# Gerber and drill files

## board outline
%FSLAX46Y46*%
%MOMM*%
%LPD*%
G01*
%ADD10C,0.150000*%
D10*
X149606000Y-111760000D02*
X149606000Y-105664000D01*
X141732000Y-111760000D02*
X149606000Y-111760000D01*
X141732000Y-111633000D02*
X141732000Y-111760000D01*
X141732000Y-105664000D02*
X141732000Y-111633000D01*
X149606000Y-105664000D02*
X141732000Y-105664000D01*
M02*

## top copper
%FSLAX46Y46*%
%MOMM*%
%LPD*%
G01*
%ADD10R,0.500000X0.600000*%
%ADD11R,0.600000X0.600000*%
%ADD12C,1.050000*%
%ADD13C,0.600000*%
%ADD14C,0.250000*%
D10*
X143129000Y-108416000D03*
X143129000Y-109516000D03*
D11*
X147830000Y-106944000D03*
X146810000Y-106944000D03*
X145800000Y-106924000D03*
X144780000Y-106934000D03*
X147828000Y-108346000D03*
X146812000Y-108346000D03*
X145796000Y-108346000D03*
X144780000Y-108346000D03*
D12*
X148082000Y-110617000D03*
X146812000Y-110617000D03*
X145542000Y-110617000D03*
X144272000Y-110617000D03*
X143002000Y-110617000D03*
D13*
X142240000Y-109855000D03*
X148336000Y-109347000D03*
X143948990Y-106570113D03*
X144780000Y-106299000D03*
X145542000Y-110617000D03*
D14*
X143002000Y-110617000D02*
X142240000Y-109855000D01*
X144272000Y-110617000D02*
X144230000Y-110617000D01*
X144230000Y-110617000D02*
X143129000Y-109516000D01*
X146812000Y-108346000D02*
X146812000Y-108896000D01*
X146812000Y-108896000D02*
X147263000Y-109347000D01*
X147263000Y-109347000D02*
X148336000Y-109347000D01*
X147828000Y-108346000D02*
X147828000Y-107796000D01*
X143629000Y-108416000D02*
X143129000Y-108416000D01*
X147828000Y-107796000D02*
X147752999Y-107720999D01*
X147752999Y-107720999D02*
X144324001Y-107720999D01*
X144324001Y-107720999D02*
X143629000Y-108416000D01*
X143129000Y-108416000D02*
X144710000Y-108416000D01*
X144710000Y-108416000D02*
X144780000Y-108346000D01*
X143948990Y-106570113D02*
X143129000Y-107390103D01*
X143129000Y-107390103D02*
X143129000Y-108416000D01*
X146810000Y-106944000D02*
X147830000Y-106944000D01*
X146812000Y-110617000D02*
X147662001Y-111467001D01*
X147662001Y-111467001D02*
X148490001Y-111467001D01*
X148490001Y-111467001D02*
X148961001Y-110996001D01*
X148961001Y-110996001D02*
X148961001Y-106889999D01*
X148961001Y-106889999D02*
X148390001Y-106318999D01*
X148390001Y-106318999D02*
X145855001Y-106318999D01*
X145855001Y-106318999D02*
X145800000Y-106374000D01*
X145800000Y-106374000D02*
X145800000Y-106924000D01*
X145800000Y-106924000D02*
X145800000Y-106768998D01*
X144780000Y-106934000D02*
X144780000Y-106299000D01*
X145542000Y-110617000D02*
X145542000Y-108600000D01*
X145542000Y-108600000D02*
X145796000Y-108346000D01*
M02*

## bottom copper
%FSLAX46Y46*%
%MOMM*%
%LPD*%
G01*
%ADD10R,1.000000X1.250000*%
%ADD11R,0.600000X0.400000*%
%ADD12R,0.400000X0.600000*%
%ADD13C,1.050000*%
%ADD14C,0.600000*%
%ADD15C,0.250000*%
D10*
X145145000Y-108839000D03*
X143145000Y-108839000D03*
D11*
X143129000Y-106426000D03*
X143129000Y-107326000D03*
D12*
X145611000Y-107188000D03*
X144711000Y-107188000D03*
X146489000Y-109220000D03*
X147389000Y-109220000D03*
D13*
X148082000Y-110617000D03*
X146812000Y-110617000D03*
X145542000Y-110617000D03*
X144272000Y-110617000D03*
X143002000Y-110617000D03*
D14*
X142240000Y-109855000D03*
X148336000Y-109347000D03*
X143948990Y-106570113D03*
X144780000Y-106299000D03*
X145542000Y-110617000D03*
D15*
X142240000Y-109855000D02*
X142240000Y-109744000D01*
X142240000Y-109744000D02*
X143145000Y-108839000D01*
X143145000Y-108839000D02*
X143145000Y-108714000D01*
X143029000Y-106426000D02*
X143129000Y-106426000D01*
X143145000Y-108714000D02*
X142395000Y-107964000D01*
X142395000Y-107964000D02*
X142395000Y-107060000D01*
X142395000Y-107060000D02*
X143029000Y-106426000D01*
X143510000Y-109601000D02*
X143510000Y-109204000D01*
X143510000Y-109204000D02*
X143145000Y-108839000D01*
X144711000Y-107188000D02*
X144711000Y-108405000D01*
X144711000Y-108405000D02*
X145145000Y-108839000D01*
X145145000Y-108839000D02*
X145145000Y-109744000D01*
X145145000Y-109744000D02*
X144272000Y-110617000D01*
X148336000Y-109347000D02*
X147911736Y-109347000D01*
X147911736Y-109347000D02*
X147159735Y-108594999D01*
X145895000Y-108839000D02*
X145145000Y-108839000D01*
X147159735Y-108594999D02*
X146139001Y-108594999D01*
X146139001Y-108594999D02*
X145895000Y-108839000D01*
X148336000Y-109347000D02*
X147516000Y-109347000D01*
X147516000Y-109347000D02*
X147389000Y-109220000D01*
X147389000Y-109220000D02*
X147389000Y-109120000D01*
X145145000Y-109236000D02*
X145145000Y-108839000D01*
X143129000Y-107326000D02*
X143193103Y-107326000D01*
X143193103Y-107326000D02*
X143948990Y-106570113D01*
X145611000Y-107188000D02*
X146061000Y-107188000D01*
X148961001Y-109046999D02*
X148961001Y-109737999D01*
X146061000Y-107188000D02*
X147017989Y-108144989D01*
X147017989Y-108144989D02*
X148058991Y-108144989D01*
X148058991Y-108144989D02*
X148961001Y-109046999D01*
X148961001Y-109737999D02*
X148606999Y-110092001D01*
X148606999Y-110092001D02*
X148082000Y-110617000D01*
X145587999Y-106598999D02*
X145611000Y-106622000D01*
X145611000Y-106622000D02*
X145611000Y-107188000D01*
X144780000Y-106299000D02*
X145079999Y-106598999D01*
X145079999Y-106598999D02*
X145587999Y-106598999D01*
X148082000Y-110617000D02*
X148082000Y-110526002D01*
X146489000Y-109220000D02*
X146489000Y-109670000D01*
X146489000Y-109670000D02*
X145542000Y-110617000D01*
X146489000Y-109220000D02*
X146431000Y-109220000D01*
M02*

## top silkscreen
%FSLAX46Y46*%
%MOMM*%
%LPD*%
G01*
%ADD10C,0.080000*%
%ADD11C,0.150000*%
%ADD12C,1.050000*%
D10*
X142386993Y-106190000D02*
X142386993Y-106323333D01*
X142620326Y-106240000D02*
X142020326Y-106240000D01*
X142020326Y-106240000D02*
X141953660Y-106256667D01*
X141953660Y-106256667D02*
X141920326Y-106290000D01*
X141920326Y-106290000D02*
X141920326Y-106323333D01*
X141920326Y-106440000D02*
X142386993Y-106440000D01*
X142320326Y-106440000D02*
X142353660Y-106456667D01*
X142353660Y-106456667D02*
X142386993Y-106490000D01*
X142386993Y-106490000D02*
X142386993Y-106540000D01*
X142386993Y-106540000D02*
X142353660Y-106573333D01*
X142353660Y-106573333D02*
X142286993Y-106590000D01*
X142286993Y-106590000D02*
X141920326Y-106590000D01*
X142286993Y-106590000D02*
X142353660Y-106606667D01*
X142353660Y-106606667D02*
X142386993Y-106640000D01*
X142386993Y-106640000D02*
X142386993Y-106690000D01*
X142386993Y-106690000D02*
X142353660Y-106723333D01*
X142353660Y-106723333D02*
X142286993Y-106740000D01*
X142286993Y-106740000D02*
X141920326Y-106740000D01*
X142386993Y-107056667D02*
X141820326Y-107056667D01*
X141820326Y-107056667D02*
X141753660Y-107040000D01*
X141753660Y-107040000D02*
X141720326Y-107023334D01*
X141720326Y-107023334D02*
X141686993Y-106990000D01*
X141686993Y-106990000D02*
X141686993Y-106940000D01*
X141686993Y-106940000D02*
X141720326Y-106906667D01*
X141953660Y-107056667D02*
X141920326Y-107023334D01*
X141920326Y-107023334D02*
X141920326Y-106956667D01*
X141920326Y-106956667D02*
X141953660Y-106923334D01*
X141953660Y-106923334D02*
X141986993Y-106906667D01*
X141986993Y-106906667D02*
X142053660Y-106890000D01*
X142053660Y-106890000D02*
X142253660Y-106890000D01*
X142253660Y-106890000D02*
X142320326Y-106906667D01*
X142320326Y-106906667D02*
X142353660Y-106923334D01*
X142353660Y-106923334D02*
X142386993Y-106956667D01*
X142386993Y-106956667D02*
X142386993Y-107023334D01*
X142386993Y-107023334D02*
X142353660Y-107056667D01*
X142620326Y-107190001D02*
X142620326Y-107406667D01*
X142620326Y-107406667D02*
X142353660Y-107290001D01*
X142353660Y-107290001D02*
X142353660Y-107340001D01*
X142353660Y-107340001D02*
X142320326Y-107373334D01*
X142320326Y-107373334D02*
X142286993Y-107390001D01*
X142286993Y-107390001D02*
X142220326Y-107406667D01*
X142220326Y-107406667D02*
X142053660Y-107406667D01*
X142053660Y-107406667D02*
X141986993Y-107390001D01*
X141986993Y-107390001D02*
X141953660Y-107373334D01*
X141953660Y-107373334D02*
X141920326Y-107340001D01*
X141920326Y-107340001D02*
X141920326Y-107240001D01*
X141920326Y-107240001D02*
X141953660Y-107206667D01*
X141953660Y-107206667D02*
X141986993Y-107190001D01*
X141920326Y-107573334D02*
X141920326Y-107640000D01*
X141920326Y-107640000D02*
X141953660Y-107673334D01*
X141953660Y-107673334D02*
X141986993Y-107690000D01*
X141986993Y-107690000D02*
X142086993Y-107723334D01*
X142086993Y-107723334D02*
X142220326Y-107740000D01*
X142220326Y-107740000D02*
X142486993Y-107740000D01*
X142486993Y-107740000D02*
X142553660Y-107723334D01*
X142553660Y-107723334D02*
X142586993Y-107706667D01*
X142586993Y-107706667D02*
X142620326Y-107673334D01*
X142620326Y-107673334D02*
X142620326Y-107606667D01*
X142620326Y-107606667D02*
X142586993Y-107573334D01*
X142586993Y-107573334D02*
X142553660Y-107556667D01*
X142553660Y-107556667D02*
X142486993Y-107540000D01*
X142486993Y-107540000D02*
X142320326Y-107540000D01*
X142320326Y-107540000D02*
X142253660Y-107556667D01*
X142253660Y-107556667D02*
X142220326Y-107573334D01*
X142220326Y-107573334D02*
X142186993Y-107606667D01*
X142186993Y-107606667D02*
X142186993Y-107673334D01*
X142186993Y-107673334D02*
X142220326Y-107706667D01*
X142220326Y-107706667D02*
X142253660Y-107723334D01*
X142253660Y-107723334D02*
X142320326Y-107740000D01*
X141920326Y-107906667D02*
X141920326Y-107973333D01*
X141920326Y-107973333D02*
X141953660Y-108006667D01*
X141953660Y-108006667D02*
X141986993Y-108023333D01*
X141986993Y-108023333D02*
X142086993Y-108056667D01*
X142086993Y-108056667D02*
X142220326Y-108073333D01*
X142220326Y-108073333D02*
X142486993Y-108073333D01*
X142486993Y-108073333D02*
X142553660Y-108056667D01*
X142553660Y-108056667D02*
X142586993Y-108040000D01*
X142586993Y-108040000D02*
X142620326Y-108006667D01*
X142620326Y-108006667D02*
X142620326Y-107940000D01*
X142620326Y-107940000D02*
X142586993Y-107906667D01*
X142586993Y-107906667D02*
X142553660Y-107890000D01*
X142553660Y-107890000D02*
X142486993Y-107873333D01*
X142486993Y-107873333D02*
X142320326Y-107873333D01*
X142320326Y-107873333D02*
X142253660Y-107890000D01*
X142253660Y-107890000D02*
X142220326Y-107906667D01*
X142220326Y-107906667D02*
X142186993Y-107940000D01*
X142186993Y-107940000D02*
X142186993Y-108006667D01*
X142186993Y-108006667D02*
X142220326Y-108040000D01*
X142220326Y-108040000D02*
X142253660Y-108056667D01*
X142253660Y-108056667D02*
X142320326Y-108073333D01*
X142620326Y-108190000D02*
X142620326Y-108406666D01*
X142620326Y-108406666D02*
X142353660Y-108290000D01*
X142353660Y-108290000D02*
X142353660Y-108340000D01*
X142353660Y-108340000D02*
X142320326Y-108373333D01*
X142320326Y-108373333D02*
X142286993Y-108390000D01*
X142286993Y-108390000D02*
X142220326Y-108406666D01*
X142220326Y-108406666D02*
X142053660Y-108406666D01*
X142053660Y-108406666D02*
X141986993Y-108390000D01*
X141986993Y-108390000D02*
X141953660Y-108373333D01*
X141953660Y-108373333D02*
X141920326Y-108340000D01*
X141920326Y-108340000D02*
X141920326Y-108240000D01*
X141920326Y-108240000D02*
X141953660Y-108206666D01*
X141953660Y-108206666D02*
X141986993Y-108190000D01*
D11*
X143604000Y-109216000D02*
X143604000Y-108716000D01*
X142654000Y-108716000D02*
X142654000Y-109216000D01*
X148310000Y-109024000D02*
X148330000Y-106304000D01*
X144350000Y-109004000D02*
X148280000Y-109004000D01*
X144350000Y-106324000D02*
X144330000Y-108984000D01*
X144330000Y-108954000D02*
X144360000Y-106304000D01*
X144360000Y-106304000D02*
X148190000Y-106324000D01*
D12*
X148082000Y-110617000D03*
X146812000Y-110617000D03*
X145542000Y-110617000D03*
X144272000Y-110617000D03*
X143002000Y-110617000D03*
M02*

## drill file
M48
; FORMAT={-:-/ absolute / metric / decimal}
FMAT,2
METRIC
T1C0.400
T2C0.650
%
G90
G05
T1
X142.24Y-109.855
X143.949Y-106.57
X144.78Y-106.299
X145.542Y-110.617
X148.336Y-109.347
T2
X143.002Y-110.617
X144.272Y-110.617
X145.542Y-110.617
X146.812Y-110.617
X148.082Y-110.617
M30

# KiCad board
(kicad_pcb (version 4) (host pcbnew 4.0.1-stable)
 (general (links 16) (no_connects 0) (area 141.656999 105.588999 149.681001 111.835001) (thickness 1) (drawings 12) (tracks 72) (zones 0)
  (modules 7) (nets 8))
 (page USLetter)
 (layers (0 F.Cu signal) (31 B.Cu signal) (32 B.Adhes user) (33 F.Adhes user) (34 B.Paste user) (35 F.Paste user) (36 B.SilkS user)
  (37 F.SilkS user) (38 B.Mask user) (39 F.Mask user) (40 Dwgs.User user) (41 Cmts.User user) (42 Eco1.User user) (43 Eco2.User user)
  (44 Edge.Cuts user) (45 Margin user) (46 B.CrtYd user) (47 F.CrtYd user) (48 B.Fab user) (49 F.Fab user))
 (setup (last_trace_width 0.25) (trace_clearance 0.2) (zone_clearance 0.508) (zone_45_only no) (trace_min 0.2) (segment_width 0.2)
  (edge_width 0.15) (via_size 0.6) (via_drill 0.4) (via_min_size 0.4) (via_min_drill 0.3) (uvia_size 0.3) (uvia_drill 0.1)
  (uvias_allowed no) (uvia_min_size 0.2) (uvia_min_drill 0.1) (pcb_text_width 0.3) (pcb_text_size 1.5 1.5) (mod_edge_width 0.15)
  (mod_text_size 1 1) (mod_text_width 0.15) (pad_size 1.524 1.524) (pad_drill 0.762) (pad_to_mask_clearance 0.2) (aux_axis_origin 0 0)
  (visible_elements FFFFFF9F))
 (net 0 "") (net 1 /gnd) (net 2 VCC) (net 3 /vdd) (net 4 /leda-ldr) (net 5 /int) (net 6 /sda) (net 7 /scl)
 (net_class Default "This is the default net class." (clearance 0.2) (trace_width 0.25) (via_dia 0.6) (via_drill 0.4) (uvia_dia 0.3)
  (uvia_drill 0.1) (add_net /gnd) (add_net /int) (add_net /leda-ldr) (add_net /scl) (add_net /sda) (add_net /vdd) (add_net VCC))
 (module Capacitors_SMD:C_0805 (layer B.Cu) (at 144.145 108.839 180)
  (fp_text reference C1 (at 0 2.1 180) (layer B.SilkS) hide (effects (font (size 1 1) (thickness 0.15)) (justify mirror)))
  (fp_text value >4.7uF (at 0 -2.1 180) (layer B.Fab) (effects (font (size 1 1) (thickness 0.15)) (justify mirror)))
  (pad 1 smd rect (at -1 0 180) (size 1 1.25) (layers B.Cu B.Paste B.Mask) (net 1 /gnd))
  (pad 2 smd rect (at 1 0 180) (size 1 1.25) (layers B.Cu B.Paste B.Mask) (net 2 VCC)))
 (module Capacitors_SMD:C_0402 (layer F.Cu) (at 143.129 108.966 270)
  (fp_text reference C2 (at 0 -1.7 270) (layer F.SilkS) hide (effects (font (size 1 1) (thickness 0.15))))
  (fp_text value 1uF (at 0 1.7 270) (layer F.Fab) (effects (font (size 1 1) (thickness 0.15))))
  (fp_line (start 0.25 -0.475) (end -0.25 -0.475) (layer F.SilkS) (width 0.15))
  (fp_line (start -0.25 0.475) (end 0.25 0.475) (layer F.SilkS) (width 0.15))
  (pad 1 smd rect (at -0.55 0 270) (size 0.6 0.5) (layers F.Cu F.Paste F.Mask) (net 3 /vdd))
  (pad 2 smd rect (at 0.55 0 270) (size 0.6 0.5) (layers F.Cu F.Paste F.Mask) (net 1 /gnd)))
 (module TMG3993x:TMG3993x (layer F.Cu) (at 143.51 107.584 90)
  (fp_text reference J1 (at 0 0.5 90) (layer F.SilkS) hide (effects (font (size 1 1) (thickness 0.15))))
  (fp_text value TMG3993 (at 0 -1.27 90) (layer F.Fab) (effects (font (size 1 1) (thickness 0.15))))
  (fp_line (start -1.44 4.8) (end 1.28 4.82) (layer F.SilkS) (width 0.15))
  (fp_line (start -1.42 0.84) (end -1.42 4.77) (layer F.SilkS) (width 0.15))
  (fp_line (start 1.26 0.84) (end -1.4 0.82) (layer F.SilkS) (width 0.15))
  (fp_line (start -1.37 0.82) (end 1.28 0.85) (layer F.SilkS) (width 0.15))
  (fp_line (start 1.28 0.85) (end 1.26 4.68) (layer F.SilkS) (width 0.15))
  (pad 5 smd rect (at 0.64 4.32 90) (size 0.6 0.6) (layers F.Cu F.Paste F.Mask) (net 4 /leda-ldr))
  (pad 6 smd rect (at 0.64 3.3 90) (size 0.6 0.6) (layers F.Cu F.Paste F.Mask) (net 4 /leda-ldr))
  (pad 7 smd rect (at 0.66 2.29 90) (size 0.6 0.6) (layers F.Cu F.Paste F.Mask) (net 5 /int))
  (pad 8 smd rect (at 0.65 1.27 90) (size 0.6 0.6) (layers F.Cu F.Paste F.Mask) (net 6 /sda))
  (pad 4 smd rect (at -0.762 4.318 90) (size 0.6 0.6) (layers F.Cu F.Paste F.Mask) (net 3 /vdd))
  (pad 3 smd rect (at -0.762 3.302 90) (size 0.6 0.6) (layers F.Cu F.Paste F.Mask) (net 1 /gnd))
  (pad 2 smd rect (at -0.762 2.286 90) (size 0.6 0.6) (layers F.Cu F.Paste F.Mask) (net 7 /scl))
  (pad 1 smd rect (at -0.762 1.27 90) (size 0.6 0.6) (layers F.Cu F.Paste F.Mask) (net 3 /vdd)))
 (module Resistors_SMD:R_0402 (layer B.Cu) (at 143.129 106.876 270)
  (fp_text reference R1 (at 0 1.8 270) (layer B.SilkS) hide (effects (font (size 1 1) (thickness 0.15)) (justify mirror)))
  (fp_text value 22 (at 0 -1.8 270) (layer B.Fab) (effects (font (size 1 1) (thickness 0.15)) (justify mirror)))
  (pad 1 smd rect (at -0.45 0 270) (size 0.4 0.6) (layers B.Cu B.Paste B.Mask) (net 2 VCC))
  (pad 2 smd rect (at 0.45 0 270) (size 0.4 0.6) (layers B.Cu B.Paste B.Mask) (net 3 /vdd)))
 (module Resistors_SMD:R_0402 (layer B.Cu) (at 145.161 107.188 180)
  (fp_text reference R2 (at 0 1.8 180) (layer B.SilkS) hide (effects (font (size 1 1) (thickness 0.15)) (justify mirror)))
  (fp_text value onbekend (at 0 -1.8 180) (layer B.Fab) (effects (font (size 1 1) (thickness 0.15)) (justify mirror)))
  (pad 1 smd rect (at -0.45 0 180) (size 0.4 0.6) (layers B.Cu B.Paste B.Mask) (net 6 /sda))
  (pad 2 smd rect (at 0.45 0 180) (size 0.4 0.6) (layers B.Cu B.Paste B.Mask) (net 1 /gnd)))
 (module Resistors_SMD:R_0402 (layer B.Cu) (at 146.939 109.22)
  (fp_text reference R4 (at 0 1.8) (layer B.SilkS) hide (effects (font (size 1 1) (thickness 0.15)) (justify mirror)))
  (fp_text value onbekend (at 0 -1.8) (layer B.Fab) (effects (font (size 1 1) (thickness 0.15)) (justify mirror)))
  (pad 1 smd rect (at -0.45 0) (size 0.4 0.6) (layers B.Cu B.Paste B.Mask) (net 7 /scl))
  (pad 2 smd rect (at 0.45 0) (size 0.4 0.6) (layers B.Cu B.Paste B.Mask) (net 1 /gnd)))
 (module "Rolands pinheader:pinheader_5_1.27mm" (layer F.Cu) (at 145.542 110.617 180)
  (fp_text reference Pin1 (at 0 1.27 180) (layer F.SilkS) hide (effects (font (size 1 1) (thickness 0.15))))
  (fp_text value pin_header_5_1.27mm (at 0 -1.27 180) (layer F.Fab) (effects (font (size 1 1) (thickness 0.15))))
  (pad 1 thru_hole circle (at -2.54 0 180) (size 1.05 1.05) (drill 0.65) (layers *.Cu *.Mask F.SilkS) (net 6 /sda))
  (pad 2 thru_hole circle (at -1.27 0 180) (size 1.05 1.05) (drill 0.65) (layers *.Cu *.Mask F.SilkS) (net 5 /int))
  (pad 3 thru_hole circle (at 0 0 180) (size 1.05 1.05) (drill 0.65) (layers *.Cu *.Mask F.SilkS) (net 7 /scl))
  (pad 4 thru_hole circle (at 1.27 0 180) (size 1.05 1.05) (drill 0.65) (layers *.Cu *.Mask F.SilkS) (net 1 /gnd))
  (pad 5 thru_hole circle (at 2.54 0 180) (size 1.05 1.05) (drill 0.65) (layers *.Cu *.Mask F.SilkS) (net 2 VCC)))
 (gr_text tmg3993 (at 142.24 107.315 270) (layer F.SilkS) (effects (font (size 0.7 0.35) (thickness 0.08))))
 (gr_line (start 149.606 111.76) (end 149.606 105.664) (layer Edge.Cuts) (width 0.15))
 (gr_line (start 141.732 111.76) (end 149.606 111.76) (layer Edge.Cuts) (width 0.15))
 (gr_line (start 141.732 111.633) (end 141.732 111.76) (layer Edge.Cuts) (width 0.15))
 (gr_line (start 141.732 105.664) (end 141.732 111.633) (layer Edge.Cuts) (width 0.15))
 (gr_line (start 149.606 105.664) (end 141.732 105.664) (layer Edge.Cuts) (width 0.15))
 (segment (start 142.24 109.855) (end 142.24 109.744) (width 0.25) (layer B.Cu) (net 2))
 (segment (start 142.24 109.744) (end 143.145 108.839) (width 0.25) (layer B.Cu) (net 2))
 (segment (start 143.002 110.617) (end 142.24 109.855) (width 0.25) (layer F.Cu) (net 2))
 (via (at 142.24 109.855) (size 0.6) (drill 0.4) (layers F.Cu B.Cu) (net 2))
 (segment (start 143.145 108.839) (end 143.145 108.714) (width 0.25) (layer B.Cu) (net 2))
 (segment (start 143.029 106.426) (end 143.129 106.426) (width 0.25) (layer B.Cu) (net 2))
 (segment (start 143.145 108.714) (end 142.395 107.964) (width 0.25) (layer B.Cu) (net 2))
 (segment (start 142.395 107.964) (end 142.395 107.06) (width 0.25) (layer B.Cu) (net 2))
 (segment (start 142.395 107.06) (end 143.029 106.426) (width 0.25) (layer B.Cu) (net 2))
 (segment (start 143.51 109.601) (end 143.51 109.204) (width 0.25) (layer B.Cu) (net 2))
 (segment (start 143.51 109.204) (end 143.145 108.839) (width 0.25) (layer B.Cu) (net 2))
 (segment (start 144.272 110.617) (end 144.23 110.617) (width 0.25) (layer F.Cu) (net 1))
 (segment (start 144.23 110.617) (end 143.129 109.516) (width 0.25) (layer F.Cu) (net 1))
 (segment (start 144.711 107.188) (end 144.711 108.405) (width 0.25) (layer B.Cu) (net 1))
 (segment (start 144.711 108.405) (end 145.145 108.839) (width 0.25) (layer B.Cu) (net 1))
 (segment (start 145.145 108.839) (end 145.145 109.744) (width 0.25) (layer B.Cu) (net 1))
 (segment (start 145.145 109.744) (end 144.272 110.617) (width 0.25) (layer B.Cu) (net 1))
 (segment (start 148.336 109.347) (end 147.911736 109.347) (width 0.25) (layer B.Cu) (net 1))
 (segment (start 147.911736 109.347) (end 147.159735 108.594999) (width 0.25) (layer B.Cu) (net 1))
 (segment (start 145.895 108.839) (end 145.145 108.839) (width 0.25) (layer B.Cu) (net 1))
 (segment (start 147.159735 108.594999) (end 146.139001 108.594999) (width 0.25) (layer B.Cu) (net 1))
 (segment (start 146.139001 108.594999) (end 145.895 108.839) (width 0.25) (layer B.Cu) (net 1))
 (segment (start 148.336 109.347) (end 147.516 109.347) (width 0.25) (layer B.Cu) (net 1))
 (segment (start 147.516 109.347) (end 147.389 109.22) (width 0.25) (layer B.Cu) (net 1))
 (segment (start 146.812 108.346) (end 146.812 108.896) (width 0.25) (layer F.Cu) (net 1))
 (segment (start 146.812 108.896) (end 147.263 109.347) (width 0.25) (layer F.Cu) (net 1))
 (segment (start 147.263 109.347) (end 148.336 109.347) (width 0.25) (layer F.Cu) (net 1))
 (via (at 148.336 109.347) (size 0.6) (drill 0.4) (layers F.Cu B.Cu) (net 1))
 (segment (start 147.389 109.22) (end 147.389 109.12) (width 0.25) (layer B.Cu) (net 1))
 (segment (start 145.145 109.236) (end 145.145 108.839) (width 0.25) (layer B.Cu) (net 1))
 (segment (start 147.828 108.346) (end 147.828 107.796) (width 0.25) (layer F.Cu) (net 3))
 (segment (start 143.629 108.416) (end 143.129 108.416) (width 0.25) (layer F.Cu) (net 3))
 (segment (start 147.828 107.796) (end 147.752999 107.720999) (width 0.25) (layer F.Cu) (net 3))
 (segment (start 147.752999 107.720999) (end 144.324001 107.720999) (width 0.25) (layer F.Cu) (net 3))
 (segment (start 144.324001 107.720999) (end 143.629 108.416) (width 0.25) (layer F.Cu) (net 3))
 (segment (start 143.129 108.416) (end 144.71 108.416) (width 0.25) (layer F.Cu) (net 3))
 (segment (start 144.71 108.416) (end 144.78 108.346) (width 0.25) (layer F.Cu) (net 3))
 (segment (start 143.94899 106.570113) (end 143.129 107.390103) (width 0.25) (layer F.Cu) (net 3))
 (segment (start 143.129 107.390103) (end 143.129 108.416) (width 0.25) (layer F.Cu) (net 3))
 (segment (start 143.129 107.326) (end 143.193103 107.326) (width 0.25) (layer B.Cu) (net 3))
 (segment (start 143.193103 107.326) (end 143.94899 106.570113) (width 0.25) (layer B.Cu) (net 3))
 (via (at 143.94899 106.570113) (size 0.6) (drill 0.4) (layers F.Cu B.Cu) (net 3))
 (segment (start 146.81 106.944) (end 147.83 106.944) (width 0.25) (layer F.Cu) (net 4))
 (segment (start 146.812 110.617) (end 147.662001 111.467001) (width 0.25) (layer F.Cu) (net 5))
 (segment (start 147.662001 111.467001) (end 148.490001 111.467001) (width 0.25) (layer F.Cu) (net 5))
 (segment (start 148.490001 111.467001) (end 148.961001 110.996001) (width 0.25) (layer F.Cu) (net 5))
 (segment (start 148.961001 110.996001) (end 148.961001 106.889999) (width 0.25) (layer F.Cu) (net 5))
 (segment (start 148.961001 106.889999) (end 148.390001 106.318999) (width 0.25) (layer F.Cu) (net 5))
 (segment (start 148.390001 106.318999) (end 145.855001 106.318999) (width 0.25) (layer F.Cu) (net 5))
 (segment (start 145.855001 106.318999) (end 145.8 106.374) (width 0.25) (layer F.Cu) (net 5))
 (segment (start 145.8 106.374) (end 145.8 106.924) (width 0.25) (layer F.Cu) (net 5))
 (segment (start 145.8 106.924) (end 145.8 106.768998) (width 0.25) (layer F.Cu) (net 5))
 (segment (start 145.611 107.188) (end 146.061 107.188) (width 0.25) (layer B.Cu) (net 6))
 (segment (start 148.961001 109.046999) (end 148.961001 109.737999) (width 0.25) (layer B.Cu) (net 6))
 (segment (start 146.061 107.188) (end 147.017989 108.144989) (width 0.25) (layer B.Cu) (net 6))
 (segment (start 147.017989 108.144989) (end 148.058991 108.144989) (width 0.25) (layer B.Cu) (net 6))
 (segment (start 148.058991 108.144989) (end 148.961001 109.046999) (width 0.25) (layer B.Cu) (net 6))
 (segment (start 148.961001 109.737999) (end 148.606999 110.092001) (width 0.25) (layer B.Cu) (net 6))
 (segment (start 148.606999 110.092001) (end 148.082 110.617) (width 0.25) (layer B.Cu) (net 6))
 (segment (start 145.587999 106.598999) (end 145.611 106.622) (width 0.25) (layer B.Cu) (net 6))
 (segment (start 145.611 106.622) (end 145.611 107.188) (width 0.25) (layer B.Cu) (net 6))
 (segment (start 144.78 106.299) (end 145.079999 106.598999) (width 0.25) (layer B.Cu) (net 6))
 (segment (start 145.079999 106.598999) (end 145.587999 106.598999) (width 0.25) (layer B.Cu) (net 6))
 (segment (start 144.78 106.934) (end 144.78 106.299) (width 0.25) (layer F.Cu) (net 6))
 (via (at 144.78 106.299) (size 0.6) (drill 0.4) (layers F.Cu B.Cu) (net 6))
 (segment (start 148.082 110.617) (end 148.082 110.526002) (width 0.25) (layer B.Cu) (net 6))
 (segment (start 145.542 110.617) (end 145.542 108.6) (width 0.25) (layer F.Cu) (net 7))
 (segment (start 145.542 108.6) (end 145.796 108.346) (width 0.25) (layer F.Cu) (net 7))
 (via (at 145.542 110.617) (size 0.6) (drill 0.4) (layers F.Cu B.Cu) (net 7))
 (segment (start 146.489 109.22) (end 146.489 109.67) (width 0.25) (layer B.Cu) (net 7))
 (segment (start 146.489 109.67) (end 145.542 110.617) (width 0.25) (layer B.Cu) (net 7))
 (segment (start 146.489 109.22) (end 146.431 109.22) (width 0.25) (layer B.Cu) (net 7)))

